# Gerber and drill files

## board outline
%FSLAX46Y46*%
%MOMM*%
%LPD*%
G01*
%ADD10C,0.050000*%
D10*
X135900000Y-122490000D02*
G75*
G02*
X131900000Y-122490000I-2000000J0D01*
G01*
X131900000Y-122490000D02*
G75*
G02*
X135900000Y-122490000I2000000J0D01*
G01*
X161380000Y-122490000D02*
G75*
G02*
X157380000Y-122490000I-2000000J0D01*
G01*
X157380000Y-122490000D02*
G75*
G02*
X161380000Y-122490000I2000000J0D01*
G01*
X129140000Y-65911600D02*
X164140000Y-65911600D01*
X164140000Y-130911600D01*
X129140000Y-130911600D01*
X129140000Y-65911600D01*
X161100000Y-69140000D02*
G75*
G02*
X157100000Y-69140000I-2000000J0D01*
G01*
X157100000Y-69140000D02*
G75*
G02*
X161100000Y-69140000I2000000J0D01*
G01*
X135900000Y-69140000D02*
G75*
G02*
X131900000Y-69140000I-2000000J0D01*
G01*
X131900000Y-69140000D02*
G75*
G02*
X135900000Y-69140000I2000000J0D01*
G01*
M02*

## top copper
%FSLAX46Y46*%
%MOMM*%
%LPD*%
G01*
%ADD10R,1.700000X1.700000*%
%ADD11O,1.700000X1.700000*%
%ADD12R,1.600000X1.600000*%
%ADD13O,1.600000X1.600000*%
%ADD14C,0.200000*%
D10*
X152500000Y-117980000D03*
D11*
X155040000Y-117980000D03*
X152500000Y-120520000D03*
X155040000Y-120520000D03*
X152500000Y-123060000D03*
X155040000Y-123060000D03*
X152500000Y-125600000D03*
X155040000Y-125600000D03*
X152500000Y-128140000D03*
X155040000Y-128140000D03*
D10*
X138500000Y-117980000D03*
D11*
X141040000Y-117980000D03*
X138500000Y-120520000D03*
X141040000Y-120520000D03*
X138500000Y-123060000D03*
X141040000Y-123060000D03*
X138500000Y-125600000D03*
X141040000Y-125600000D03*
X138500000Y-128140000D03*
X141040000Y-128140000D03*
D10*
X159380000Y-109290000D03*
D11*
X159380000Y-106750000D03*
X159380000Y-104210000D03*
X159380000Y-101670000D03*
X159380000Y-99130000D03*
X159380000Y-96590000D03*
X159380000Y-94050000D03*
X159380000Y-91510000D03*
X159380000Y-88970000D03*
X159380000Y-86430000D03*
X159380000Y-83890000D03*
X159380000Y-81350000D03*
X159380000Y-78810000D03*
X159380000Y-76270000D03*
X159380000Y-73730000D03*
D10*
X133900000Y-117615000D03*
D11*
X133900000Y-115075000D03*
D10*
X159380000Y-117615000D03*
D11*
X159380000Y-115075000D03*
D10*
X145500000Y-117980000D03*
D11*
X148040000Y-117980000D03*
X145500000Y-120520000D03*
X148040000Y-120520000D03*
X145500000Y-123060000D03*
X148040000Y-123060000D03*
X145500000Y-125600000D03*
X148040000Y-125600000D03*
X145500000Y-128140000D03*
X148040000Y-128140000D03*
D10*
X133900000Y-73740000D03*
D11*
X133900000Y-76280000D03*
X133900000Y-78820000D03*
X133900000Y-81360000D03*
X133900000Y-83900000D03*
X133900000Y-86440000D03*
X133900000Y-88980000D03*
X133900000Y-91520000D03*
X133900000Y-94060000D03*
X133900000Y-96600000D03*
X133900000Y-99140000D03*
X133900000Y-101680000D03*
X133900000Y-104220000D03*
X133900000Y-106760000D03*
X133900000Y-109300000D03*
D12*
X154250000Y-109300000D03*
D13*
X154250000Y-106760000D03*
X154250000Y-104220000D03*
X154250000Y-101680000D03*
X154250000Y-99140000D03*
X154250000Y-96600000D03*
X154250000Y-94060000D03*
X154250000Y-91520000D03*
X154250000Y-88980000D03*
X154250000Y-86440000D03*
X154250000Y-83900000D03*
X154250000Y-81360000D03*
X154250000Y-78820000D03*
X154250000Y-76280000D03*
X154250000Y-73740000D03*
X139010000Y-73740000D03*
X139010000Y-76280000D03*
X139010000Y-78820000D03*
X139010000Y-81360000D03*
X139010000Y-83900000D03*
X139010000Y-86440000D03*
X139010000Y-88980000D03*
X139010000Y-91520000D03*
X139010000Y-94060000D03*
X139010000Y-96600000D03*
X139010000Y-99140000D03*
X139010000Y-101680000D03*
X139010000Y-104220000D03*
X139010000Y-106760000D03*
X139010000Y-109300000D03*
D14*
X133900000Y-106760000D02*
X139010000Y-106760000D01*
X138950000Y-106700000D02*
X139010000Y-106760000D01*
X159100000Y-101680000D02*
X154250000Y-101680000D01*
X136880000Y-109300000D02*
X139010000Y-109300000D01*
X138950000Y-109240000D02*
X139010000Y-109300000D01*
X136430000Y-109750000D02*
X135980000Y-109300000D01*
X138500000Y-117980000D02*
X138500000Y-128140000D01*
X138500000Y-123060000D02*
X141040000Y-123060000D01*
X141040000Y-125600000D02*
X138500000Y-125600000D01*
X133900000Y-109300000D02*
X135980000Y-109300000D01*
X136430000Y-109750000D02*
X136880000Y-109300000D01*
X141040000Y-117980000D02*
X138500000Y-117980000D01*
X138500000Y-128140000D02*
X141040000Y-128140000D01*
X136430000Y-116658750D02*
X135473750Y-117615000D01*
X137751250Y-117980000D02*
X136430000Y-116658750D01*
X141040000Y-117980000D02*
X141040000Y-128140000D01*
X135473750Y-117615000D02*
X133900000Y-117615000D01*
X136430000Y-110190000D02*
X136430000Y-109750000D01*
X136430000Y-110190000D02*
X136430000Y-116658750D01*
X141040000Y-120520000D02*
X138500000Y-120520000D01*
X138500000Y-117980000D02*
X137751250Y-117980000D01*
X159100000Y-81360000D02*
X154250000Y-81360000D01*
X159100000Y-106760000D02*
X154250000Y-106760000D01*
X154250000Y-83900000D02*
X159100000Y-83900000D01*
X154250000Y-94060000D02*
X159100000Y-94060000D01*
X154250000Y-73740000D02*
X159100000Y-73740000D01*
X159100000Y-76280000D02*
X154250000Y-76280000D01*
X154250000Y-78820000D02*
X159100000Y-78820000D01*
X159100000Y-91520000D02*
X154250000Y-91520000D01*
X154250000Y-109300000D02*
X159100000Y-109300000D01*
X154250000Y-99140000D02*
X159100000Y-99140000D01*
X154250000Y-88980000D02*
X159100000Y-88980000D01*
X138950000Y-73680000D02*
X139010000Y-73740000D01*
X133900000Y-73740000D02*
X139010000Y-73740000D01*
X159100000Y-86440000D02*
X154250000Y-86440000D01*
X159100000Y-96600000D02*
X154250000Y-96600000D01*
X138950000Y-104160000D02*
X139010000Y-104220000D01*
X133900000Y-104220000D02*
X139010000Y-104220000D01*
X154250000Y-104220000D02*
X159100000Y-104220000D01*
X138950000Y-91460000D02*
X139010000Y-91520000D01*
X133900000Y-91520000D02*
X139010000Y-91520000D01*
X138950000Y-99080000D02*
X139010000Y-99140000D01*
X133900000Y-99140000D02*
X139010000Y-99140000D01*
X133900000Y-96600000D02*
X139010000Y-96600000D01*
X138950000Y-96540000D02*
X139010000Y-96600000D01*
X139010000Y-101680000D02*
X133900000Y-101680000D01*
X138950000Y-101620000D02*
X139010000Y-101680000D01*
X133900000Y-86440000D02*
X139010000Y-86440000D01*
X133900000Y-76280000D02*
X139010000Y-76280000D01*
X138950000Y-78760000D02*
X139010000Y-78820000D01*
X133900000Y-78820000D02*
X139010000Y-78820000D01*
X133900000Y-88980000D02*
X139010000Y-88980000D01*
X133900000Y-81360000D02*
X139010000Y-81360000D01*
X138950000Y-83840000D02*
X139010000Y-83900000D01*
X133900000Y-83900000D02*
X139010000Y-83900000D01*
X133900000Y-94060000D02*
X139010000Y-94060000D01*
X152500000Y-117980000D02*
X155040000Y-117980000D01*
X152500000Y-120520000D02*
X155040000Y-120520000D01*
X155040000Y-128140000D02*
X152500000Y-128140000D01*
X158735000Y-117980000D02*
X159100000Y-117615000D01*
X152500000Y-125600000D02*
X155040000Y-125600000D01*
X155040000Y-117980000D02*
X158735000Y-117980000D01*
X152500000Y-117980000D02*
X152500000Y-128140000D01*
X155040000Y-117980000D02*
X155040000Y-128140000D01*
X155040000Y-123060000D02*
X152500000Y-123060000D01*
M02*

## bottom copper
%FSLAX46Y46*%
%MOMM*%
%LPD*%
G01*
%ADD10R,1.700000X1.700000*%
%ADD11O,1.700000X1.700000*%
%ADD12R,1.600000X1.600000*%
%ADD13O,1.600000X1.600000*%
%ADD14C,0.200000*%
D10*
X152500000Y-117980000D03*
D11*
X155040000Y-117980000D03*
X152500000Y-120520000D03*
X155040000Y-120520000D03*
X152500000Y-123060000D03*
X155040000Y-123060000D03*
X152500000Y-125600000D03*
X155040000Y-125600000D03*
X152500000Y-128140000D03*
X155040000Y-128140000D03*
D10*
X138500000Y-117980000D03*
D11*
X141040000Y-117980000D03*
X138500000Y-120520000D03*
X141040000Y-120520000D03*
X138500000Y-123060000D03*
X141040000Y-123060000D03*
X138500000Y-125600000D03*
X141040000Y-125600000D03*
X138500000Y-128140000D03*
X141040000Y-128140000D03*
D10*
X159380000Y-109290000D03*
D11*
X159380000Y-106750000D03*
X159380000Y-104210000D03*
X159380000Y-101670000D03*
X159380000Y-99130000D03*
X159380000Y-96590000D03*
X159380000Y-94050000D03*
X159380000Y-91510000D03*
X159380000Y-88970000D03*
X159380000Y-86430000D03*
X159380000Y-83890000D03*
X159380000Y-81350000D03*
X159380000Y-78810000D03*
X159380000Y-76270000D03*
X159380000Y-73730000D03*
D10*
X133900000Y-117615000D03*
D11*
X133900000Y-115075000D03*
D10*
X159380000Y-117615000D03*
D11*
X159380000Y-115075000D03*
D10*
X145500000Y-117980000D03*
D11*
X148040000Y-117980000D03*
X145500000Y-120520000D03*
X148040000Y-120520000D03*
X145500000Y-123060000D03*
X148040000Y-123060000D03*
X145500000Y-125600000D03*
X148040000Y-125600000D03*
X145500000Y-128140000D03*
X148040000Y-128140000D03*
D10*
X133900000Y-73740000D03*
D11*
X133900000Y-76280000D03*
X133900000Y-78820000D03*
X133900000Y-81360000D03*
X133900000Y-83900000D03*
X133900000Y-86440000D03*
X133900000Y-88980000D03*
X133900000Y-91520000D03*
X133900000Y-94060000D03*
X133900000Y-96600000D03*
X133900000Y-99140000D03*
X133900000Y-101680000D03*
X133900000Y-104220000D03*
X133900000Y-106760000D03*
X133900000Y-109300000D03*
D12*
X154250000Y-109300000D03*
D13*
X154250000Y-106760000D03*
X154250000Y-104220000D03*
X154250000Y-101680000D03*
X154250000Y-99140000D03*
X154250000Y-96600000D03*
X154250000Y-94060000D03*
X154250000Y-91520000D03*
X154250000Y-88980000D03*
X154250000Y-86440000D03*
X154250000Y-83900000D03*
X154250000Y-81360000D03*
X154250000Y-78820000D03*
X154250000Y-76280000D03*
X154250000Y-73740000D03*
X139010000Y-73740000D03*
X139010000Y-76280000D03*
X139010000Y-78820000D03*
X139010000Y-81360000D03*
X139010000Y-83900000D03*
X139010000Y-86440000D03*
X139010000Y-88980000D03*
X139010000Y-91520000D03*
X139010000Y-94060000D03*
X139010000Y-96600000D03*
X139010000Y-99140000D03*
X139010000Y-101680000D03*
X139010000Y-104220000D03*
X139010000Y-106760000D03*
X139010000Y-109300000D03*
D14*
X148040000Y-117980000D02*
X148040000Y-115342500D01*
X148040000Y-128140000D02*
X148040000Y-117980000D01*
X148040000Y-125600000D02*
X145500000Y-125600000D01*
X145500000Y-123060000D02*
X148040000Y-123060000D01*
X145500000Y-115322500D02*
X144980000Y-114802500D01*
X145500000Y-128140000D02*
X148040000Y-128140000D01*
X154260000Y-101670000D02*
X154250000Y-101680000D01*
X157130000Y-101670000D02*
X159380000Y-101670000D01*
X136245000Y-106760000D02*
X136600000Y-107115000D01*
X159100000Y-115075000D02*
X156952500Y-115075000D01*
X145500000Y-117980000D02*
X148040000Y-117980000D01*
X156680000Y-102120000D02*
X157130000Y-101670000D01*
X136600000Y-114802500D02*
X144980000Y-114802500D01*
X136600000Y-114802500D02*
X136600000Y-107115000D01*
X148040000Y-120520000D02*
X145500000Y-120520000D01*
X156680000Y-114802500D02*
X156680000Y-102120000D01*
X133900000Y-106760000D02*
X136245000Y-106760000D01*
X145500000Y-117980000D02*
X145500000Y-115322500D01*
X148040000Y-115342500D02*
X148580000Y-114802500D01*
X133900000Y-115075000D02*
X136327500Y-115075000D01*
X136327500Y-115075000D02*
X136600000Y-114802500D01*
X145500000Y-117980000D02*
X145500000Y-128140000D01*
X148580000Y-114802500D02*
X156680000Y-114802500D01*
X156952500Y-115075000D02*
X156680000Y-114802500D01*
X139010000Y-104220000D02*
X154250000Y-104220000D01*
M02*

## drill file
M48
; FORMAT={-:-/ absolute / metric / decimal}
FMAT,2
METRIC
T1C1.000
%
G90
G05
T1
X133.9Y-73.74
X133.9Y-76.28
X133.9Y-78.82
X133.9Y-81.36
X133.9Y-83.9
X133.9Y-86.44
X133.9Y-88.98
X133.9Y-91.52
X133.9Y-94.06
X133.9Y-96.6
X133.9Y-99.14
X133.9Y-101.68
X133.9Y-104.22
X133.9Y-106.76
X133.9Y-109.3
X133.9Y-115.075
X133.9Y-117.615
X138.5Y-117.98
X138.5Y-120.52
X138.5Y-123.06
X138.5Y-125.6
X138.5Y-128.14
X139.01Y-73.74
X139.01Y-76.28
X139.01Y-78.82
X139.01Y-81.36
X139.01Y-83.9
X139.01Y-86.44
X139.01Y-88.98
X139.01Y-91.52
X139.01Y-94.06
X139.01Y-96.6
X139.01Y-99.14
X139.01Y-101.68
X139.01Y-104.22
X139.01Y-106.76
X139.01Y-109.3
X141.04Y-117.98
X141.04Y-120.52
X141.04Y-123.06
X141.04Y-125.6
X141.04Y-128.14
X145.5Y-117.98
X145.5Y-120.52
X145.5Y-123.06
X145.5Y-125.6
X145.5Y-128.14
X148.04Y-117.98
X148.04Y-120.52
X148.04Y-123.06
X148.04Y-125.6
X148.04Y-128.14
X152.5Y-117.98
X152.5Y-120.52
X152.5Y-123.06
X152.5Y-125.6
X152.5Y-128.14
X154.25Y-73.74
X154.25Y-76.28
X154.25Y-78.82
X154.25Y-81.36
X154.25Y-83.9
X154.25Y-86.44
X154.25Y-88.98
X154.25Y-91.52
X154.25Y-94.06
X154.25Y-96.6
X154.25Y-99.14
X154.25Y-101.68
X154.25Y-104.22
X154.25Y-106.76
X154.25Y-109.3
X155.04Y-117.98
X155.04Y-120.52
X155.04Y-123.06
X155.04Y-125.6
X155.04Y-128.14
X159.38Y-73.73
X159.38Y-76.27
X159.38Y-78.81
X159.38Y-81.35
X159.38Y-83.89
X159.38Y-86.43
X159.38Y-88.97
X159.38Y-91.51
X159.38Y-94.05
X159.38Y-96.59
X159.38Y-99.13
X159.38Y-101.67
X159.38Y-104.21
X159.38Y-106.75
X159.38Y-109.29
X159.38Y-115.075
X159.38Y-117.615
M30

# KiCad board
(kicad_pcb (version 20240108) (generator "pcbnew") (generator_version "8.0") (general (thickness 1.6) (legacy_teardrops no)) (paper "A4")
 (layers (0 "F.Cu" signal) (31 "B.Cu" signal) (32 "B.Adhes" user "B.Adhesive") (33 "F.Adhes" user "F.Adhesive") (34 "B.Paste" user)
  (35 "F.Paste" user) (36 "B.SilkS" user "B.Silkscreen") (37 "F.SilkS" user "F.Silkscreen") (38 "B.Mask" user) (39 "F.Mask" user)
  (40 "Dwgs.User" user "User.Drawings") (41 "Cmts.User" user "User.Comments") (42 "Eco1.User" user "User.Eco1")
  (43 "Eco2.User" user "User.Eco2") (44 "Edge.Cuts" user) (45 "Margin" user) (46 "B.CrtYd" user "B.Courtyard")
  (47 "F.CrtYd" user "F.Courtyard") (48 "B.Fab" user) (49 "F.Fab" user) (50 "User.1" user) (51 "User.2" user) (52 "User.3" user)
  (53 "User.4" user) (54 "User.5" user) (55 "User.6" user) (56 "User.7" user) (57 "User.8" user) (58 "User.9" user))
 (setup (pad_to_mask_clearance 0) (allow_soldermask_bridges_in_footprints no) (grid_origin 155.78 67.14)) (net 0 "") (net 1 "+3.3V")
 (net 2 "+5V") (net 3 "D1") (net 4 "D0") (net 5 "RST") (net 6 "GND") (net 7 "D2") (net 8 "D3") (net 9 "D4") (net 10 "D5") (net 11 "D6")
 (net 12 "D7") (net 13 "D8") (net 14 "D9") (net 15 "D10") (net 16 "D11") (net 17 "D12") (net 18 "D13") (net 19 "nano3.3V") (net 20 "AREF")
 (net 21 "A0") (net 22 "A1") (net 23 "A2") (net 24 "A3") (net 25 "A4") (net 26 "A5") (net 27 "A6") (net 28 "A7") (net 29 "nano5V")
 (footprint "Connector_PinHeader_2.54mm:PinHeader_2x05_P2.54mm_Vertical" (layer "F.Cu") (at 152.5 117.98)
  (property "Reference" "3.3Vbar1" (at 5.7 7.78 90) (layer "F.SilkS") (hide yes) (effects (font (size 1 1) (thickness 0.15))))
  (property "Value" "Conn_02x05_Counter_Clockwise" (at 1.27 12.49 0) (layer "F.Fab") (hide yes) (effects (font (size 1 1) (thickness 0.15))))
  (pad "1" thru_hole rect (at 0 0) (size 1.7 1.7) (drill 1) (layers "*.Cu" "*.Mask") (remove_unused_layers no) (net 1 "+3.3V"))
  (pad "2" thru_hole oval (at 2.54 0) (size 1.7 1.7) (drill 1) (layers "*.Cu" "*.Mask") (remove_unused_layers no) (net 1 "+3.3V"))
  (pad "3" thru_hole oval (at 0 2.54) (size 1.7 1.7) (drill 1) (layers "*.Cu" "*.Mask") (remove_unused_layers no) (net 1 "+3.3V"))
  (pad "4" thru_hole oval (at 2.54 2.54) (size 1.7 1.7) (drill 1) (layers "*.Cu" "*.Mask") (remove_unused_layers no) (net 1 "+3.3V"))
  (pad "5" thru_hole oval (at 0 5.08) (size 1.7 1.7) (drill 1) (layers "*.Cu" "*.Mask") (remove_unused_layers no) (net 1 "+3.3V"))
  (pad "6" thru_hole oval (at 2.54 5.08) (size 1.7 1.7) (drill 1) (layers "*.Cu" "*.Mask") (remove_unused_layers no) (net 1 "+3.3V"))
  (pad "7" thru_hole oval (at 0 7.62) (size 1.7 1.7) (drill 1) (layers "*.Cu" "*.Mask") (remove_unused_layers no) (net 1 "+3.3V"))
  (pad "8" thru_hole oval (at 2.54 7.62) (size 1.7 1.7) (drill 1) (layers "*.Cu" "*.Mask") (remove_unused_layers no) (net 1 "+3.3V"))
  (pad "9" thru_hole oval (at 0 10.16) (size 1.7 1.7) (drill 1) (layers "*.Cu" "*.Mask") (remove_unused_layers no) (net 1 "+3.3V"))
  (pad "10" thru_hole oval (at 2.54 10.16) (size 1.7 1.7) (drill 1) (layers "*.Cu" "*.Mask") (remove_unused_layers no) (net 1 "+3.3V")))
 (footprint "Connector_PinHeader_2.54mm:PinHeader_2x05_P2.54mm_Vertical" (layer "F.Cu") (at 138.5 117.98)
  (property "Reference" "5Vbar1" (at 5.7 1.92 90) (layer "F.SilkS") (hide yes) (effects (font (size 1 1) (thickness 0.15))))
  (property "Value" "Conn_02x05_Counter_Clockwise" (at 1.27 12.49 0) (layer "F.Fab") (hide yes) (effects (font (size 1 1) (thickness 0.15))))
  (pad "1" thru_hole rect (at 0 0) (size 1.7 1.7) (drill 1) (layers "*.Cu" "*.Mask") (remove_unused_layers no) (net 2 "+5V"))
  (pad "2" thru_hole oval (at 2.54 0) (size 1.7 1.7) (drill 1) (layers "*.Cu" "*.Mask") (remove_unused_layers no) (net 2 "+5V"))
  (pad "3" thru_hole oval (at 0 2.54) (size 1.7 1.7) (drill 1) (layers "*.Cu" "*.Mask") (remove_unused_layers no) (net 2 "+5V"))
  (pad "4" thru_hole oval (at 2.54 2.54) (size 1.7 1.7) (drill 1) (layers "*.Cu" "*.Mask") (remove_unused_layers no) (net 2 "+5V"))
  (pad "5" thru_hole oval (at 0 5.08) (size 1.7 1.7) (drill 1) (layers "*.Cu" "*.Mask") (remove_unused_layers no) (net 2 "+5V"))
  (pad "6" thru_hole oval (at 2.54 5.08) (size 1.7 1.7) (drill 1) (layers "*.Cu" "*.Mask") (remove_unused_layers no) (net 2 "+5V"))
  (pad "7" thru_hole oval (at 0 7.62) (size 1.7 1.7) (drill 1) (layers "*.Cu" "*.Mask") (remove_unused_layers no) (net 2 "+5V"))
  (pad "8" thru_hole oval (at 2.54 7.62) (size 1.7 1.7) (drill 1) (layers "*.Cu" "*.Mask") (remove_unused_layers no) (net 2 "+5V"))
  (pad "9" thru_hole oval (at 0 10.16) (size 1.7 1.7) (drill 1) (layers "*.Cu" "*.Mask") (remove_unused_layers no) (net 2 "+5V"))
  (pad "10" thru_hole oval (at 2.54 10.16) (size 1.7 1.7) (drill 1) (layers "*.Cu" "*.Mask") (remove_unused_layers no) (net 2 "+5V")))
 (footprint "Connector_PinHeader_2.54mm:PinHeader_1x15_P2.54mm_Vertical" (layer "F.Cu") (at 159.38 109.29 180)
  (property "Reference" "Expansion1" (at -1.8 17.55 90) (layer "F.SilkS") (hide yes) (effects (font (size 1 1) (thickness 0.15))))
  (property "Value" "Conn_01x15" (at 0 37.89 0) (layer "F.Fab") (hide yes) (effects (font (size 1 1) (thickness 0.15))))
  (pad "1" thru_hole rect (at 0 0 180) (size 1.7 1.7) (drill 1) (layers "*.Cu" "*.Mask") (remove_unused_layers no) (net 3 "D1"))
  (pad "2" thru_hole oval (at 0 2.54 180) (size 1.7 1.7) (drill 1) (layers "*.Cu" "*.Mask") (remove_unused_layers no) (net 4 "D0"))
  (pad "3" thru_hole oval (at 0 5.08 180) (size 1.7 1.7) (drill 1) (layers "*.Cu" "*.Mask") (remove_unused_layers no) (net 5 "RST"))
  (pad "4" thru_hole oval (at 0 7.62 180) (size 1.7 1.7) (drill 1) (layers "*.Cu" "*.Mask") (remove_unused_layers no) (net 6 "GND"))
  (pad "5" thru_hole oval (at 0 10.16 180) (size 1.7 1.7) (drill 1) (layers "*.Cu" "*.Mask") (remove_unused_layers no) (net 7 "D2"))
  (pad "6" thru_hole oval (at 0 12.7 180) (size 1.7 1.7) (drill 1) (layers "*.Cu" "*.Mask") (remove_unused_layers no) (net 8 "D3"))
  (pad "7" thru_hole oval (at 0 15.24 180) (size 1.7 1.7) (drill 1) (layers "*.Cu" "*.Mask") (remove_unused_layers no) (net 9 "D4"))
  (pad "8" thru_hole oval (at 0 17.78 180) (size 1.7 1.7) (drill 1) (layers "*.Cu" "*.Mask") (remove_unused_layers no) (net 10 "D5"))
  (pad "9" thru_hole oval (at 0 20.32 180) (size 1.7 1.7) (drill 1) (layers "*.Cu" "*.Mask") (remove_unused_layers no) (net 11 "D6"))
  (pad "10" thru_hole oval (at 0 22.86 180) (size 1.7 1.7) (drill 1) (layers "*.Cu" "*.Mask") (remove_unused_layers no) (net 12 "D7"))
  (pad "11" thru_hole oval (at 0 25.4 180) (size 1.7 1.7) (drill 1) (layers "*.Cu" "*.Mask") (remove_unused_layers no) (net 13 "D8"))
  (pad "12" thru_hole oval (at 0 27.94 180) (size 1.7 1.7) (drill 1) (layers "*.Cu" "*.Mask") (remove_unused_layers no) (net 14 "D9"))
  (pad "13" thru_hole oval (at 0 30.48 180) (size 1.7 1.7) (drill 1) (layers "*.Cu" "*.Mask") (remove_unused_layers no) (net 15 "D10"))
  (pad "14" thru_hole oval (at 0 33.02 180) (size 1.7 1.7) (drill 1) (layers "*.Cu" "*.Mask") (remove_unused_layers no) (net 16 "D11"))
  (pad "15" thru_hole oval (at 0 35.56 180) (size 1.7 1.7) (drill 1) (layers "*.Cu" "*.Mask") (remove_unused_layers no) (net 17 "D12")))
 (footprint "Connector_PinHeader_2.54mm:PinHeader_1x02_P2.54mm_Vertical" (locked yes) (layer "F.Cu") (at 133.9 117.615 180)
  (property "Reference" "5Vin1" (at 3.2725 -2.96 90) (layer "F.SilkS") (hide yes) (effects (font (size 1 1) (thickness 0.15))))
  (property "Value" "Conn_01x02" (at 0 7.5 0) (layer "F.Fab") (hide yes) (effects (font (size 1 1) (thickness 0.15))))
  (pad "1" thru_hole rect (at 0 0 180) (size 1.7 1.7) (drill 1) (layers "*.Cu" "*.Mask") (remove_unused_layers no) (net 2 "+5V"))
  (pad "2" thru_hole oval (at 0 2.54 180) (size 1.7 1.7) (drill 1) (layers "*.Cu" "*.Mask") (remove_unused_layers no) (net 6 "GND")))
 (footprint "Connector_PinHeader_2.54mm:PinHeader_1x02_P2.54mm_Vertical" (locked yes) (layer "F.Cu") (at 159.38 117.615 180)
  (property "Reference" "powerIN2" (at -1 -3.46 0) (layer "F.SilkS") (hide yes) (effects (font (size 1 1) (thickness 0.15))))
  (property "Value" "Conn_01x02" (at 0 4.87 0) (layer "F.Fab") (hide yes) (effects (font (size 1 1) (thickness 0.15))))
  (pad "1" thru_hole rect (at 0 0 180) (size 1.7 1.7) (drill 1) (layers "*.Cu" "*.Mask") (remove_unused_layers no) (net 1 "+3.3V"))
  (pad "2" thru_hole oval (at 0 2.54 180) (size 1.7 1.7) (drill 1) (layers "*.Cu" "*.Mask") (remove_unused_layers no) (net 6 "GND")))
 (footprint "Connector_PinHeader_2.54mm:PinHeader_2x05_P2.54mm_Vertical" (layer "F.Cu") (at 145.5 117.98)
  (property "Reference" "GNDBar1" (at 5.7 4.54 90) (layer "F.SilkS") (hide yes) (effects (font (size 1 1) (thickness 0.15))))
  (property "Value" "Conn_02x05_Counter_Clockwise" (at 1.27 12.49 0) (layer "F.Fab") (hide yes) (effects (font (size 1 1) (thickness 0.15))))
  (pad "1" thru_hole rect (at 0 0) (size 1.7 1.7) (drill 1) (layers "*.Cu" "*.Mask") (remove_unused_layers no) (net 6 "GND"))
  (pad "2" thru_hole oval (at 2.54 0) (size 1.7 1.7) (drill 1) (layers "*.Cu" "*.Mask") (remove_unused_layers no) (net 6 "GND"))
  (pad "3" thru_hole oval (at 0 2.54) (size 1.7 1.7) (drill 1) (layers "*.Cu" "*.Mask") (remove_unused_layers no) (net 6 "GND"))
  (pad "4" thru_hole oval (at 2.54 2.54) (size 1.7 1.7) (drill 1) (layers "*.Cu" "*.Mask") (remove_unused_layers no) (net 6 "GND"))
  (pad "5" thru_hole oval (at 0 5.08) (size 1.7 1.7) (drill 1) (layers "*.Cu" "*.Mask") (remove_unused_layers no) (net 6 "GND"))
  (pad "6" thru_hole oval (at 2.54 5.08) (size 1.7 1.7) (drill 1) (layers "*.Cu" "*.Mask") (remove_unused_layers no) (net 6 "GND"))
  (pad "7" thru_hole oval (at 0 7.62) (size 1.7 1.7) (drill 1) (layers "*.Cu" "*.Mask") (remove_unused_layers no) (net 6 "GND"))
  (pad "8" thru_hole oval (at 2.54 7.62) (size 1.7 1.7) (drill 1) (layers "*.Cu" "*.Mask") (remove_unused_layers no) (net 6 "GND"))
  (pad "9" thru_hole oval (at 0 10.16) (size 1.7 1.7) (drill 1) (layers "*.Cu" "*.Mask") (remove_unused_layers no) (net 6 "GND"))
  (pad "10" thru_hole oval (at 2.54 10.16) (size 1.7 1.7) (drill 1) (layers "*.Cu" "*.Mask") (remove_unused_layers no) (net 6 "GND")))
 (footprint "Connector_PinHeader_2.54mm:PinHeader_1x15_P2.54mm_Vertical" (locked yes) (layer "F.Cu") (at 133.9 73.74)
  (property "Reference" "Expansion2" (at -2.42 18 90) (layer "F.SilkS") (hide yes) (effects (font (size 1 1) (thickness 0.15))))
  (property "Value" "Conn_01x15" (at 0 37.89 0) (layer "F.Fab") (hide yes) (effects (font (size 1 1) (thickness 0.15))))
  (pad "1" thru_hole rect (at 0 0) (size 1.7 1.7) (drill 1) (layers "*.Cu" "*.Mask") (remove_unused_layers no) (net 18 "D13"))
  (pad "2" thru_hole oval (at 0 2.54) (size 1.7 1.7) (drill 1) (layers "*.Cu" "*.Mask") (remove_unused_layers no) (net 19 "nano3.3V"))
  (pad "3" thru_hole oval (at 0 5.08) (size 1.7 1.7) (drill 1) (layers "*.Cu" "*.Mask") (remove_unused_layers no) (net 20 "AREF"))
  (pad "4" thru_hole oval (at 0 7.62) (size 1.7 1.7) (drill 1) (layers "*.Cu" "*.Mask") (remove_unused_layers no) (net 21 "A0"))
  (pad "5" thru_hole oval (at 0 10.16) (size 1.7 1.7) (drill 1) (layers "*.Cu" "*.Mask") (remove_unused_layers no) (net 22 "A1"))
  (pad "6" thru_hole oval (at 0 12.7) (size 1.7 1.7) (drill 1) (layers "*.Cu" "*.Mask") (remove_unused_layers no) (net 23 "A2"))
  (pad "7" thru_hole oval (at 0 15.24) (size 1.7 1.7) (drill 1) (layers "*.Cu" "*.Mask") (remove_unused_layers no) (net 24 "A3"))
  (pad "8" thru_hole oval (at 0 17.78) (size 1.7 1.7) (drill 1) (layers "*.Cu" "*.Mask") (remove_unused_layers no) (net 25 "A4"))
  (pad "9" thru_hole oval (at 0 20.32) (size 1.7 1.7) (drill 1) (layers "*.Cu" "*.Mask") (remove_unused_layers no) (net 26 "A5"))
  (pad "10" thru_hole oval (at 0 22.86) (size 1.7 1.7) (drill 1) (layers "*.Cu" "*.Mask") (remove_unused_layers no) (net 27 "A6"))
  (pad "11" thru_hole oval (at 0 25.4) (size 1.7 1.7) (drill 1) (layers "*.Cu" "*.Mask") (remove_unused_layers no) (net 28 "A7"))
  (pad "12" thru_hole oval (at 0 27.94) (size 1.7 1.7) (drill 1) (layers "*.Cu" "*.Mask") (remove_unused_layers no) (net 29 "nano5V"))
  (pad "13" thru_hole oval (at 0 30.48) (size 1.7 1.7) (drill 1) (layers "*.Cu" "*.Mask") (remove_unused_layers no) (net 5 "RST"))
  (pad "14" thru_hole oval (at 0 33.02) (size 1.7 1.7) (drill 1) (layers "*.Cu" "*.Mask") (remove_unused_layers no) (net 6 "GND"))
  (pad "15" thru_hole oval (at 0 35.56) (size 1.7 1.7) (drill 1) (layers "*.Cu" "*.Mask") (remove_unused_layers no) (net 2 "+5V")))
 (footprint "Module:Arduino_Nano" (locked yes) (layer "F.Cu") (at 154.25 109.3 180)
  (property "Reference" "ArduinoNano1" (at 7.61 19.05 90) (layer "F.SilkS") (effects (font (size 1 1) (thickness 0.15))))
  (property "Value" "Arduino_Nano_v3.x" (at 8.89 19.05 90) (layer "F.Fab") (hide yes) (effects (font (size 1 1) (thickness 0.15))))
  (pad "1" thru_hole rect (at 0 0 180) (size 1.6 1.6) (drill 1) (layers "*.Cu" "*.Mask") (remove_unused_layers no) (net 3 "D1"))
  (pad "2" thru_hole oval (at 0 2.54 180) (size 1.6 1.6) (drill 1) (layers "*.Cu" "*.Mask") (remove_unused_layers no) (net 4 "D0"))
  (pad "3" thru_hole oval (at 0 5.08 180) (size 1.6 1.6) (drill 1) (layers "*.Cu" "*.Mask") (remove_unused_layers no) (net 5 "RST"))
  (pad "4" thru_hole oval (at 0 7.62 180) (size 1.6 1.6) (drill 1) (layers "*.Cu" "*.Mask") (remove_unused_layers no) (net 6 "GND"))
  (pad "5" thru_hole oval (at 0 10.16 180) (size 1.6 1.6) (drill 1) (layers "*.Cu" "*.Mask") (remove_unused_layers no) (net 7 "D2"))
  (pad "6" thru_hole oval (at 0 12.7 180) (size 1.6 1.6) (drill 1) (layers "*.Cu" "*.Mask") (remove_unused_layers no) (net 8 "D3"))
  (pad "7" thru_hole oval (at 0 15.24 180) (size 1.6 1.6) (drill 1) (layers "*.Cu" "*.Mask") (remove_unused_layers no) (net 9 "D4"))
  (pad "8" thru_hole oval (at 0 17.78 180) (size 1.6 1.6) (drill 1) (layers "*.Cu" "*.Mask") (remove_unused_layers no) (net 10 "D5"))
  (pad "9" thru_hole oval (at 0 20.32 180) (size 1.6 1.6) (drill 1) (layers "*.Cu" "*.Mask") (remove_unused_layers no) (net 11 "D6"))
  (pad "10" thru_hole oval (at 0 22.86 180) (size 1.6 1.6) (drill 1) (layers "*.Cu" "*.Mask") (remove_unused_layers no) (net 12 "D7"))
  (pad "11" thru_hole oval (at 0 25.4 180) (size 1.6 1.6) (drill 1) (layers "*.Cu" "*.Mask") (remove_unused_layers no) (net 13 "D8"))
  (pad "12" thru_hole oval (at 0 27.94 180) (size 1.6 1.6) (drill 1) (layers "*.Cu" "*.Mask") (remove_unused_layers no) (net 14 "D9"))
  (pad "13" thru_hole oval (at 0 30.48 180) (size 1.6 1.6) (drill 1) (layers "*.Cu" "*.Mask") (remove_unused_layers no) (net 15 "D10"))
  (pad "14" thru_hole oval (at 0 33.02 180) (size 1.6 1.6) (drill 1) (layers "*.Cu" "*.Mask") (remove_unused_layers no) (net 16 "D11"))
  (pad "15" thru_hole oval (at 0 35.56 180) (size 1.6 1.6) (drill 1) (layers "*.Cu" "*.Mask") (remove_unused_layers no) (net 17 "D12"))
  (pad "16" thru_hole oval (at 15.24 35.56 180) (size 1.6 1.6) (drill 1) (layers "*.Cu" "*.Mask") (remove_unused_layers no) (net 18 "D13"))
  (pad "17" thru_hole oval (at 15.24 33.02 180) (size 1.6 1.6) (drill 1) (layers "*.Cu" "*.Mask") (remove_unused_layers no)
   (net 19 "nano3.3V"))
  (pad "18" thru_hole oval (at 15.24 30.48 180) (size 1.6 1.6) (drill 1) (layers "*.Cu" "*.Mask") (remove_unused_layers no) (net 20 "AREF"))
  (pad "19" thru_hole oval (at 15.24 27.94 180) (size 1.6 1.6) (drill 1) (layers "*.Cu" "*.Mask") (remove_unused_layers no) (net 21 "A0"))
  (pad "20" thru_hole oval (at 15.24 25.4 180) (size 1.6 1.6) (drill 1) (layers "*.Cu" "*.Mask") (remove_unused_layers no) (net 22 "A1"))
  (pad "21" thru_hole oval (at 15.24 22.86 180) (size 1.6 1.6) (drill 1) (layers "*.Cu" "*.Mask") (remove_unused_layers no) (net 23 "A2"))
  (pad "22" thru_hole oval (at 15.24 20.32 180) (size 1.6 1.6) (drill 1) (layers "*.Cu" "*.Mask") (remove_unused_layers no) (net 24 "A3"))
  (pad "23" thru_hole oval (at 15.24 17.78 180) (size 1.6 1.6) (drill 1) (layers "*.Cu" "*.Mask") (remove_unused_layers no) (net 25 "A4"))
  (pad "24" thru_hole oval (at 15.24 15.24 180) (size 1.6 1.6) (drill 1) (layers "*.Cu" "*.Mask") (remove_unused_layers no) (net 26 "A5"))
  (pad "25" thru_hole oval (at 15.24 12.7 180) (size 1.6 1.6) (drill 1) (layers "*.Cu" "*.Mask") (remove_unused_layers no) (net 27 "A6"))
  (pad "26" thru_hole oval (at 15.24 10.16 180) (size 1.6 1.6) (drill 1) (layers "*.Cu" "*.Mask") (remove_unused_layers no) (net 28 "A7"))
  (pad "27" thru_hole oval (at 15.24 7.62 180) (size 1.6 1.6) (drill 1) (layers "*.Cu" "*.Mask") (remove_unused_layers no) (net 29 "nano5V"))
  (pad "28" thru_hole oval (at 15.24 5.08 180) (size 1.6 1.6) (drill 1) (layers "*.Cu" "*.Mask") (remove_unused_layers no) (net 5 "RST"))
  (pad "29" thru_hole oval (at 15.24 2.54 180) (size 1.6 1.6) (drill 1) (layers "*.Cu" "*.Mask") (remove_unused_layers no) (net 6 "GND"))
  (pad "30" thru_hole oval (at 15.24 0 180) (size 1.6 1.6) (drill 1) (layers "*.Cu" "*.Mask") (remove_unused_layers no) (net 2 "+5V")))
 (gr_circle (center 133.9 122.49) (end 135.9 122.49) (stroke (width 0.05) (type default)) (fill none) (layer "Edge.Cuts"))
 (gr_circle (center 159.38 122.49) (end 161.38 122.49) (stroke (width 0.05) (type default)) (fill none) (layer "Edge.Cuts"))
 (gr_rect (start 129.14 65.9116) (end 164.14 130.9116) (stroke (width 0.05) (type default)) (fill none) (layer "Edge.Cuts"))
 (gr_circle (center 159.1 69.14) (end 161.1 69.14) (stroke (width 0.05) (type default)) (fill none) (layer "Edge.Cuts"))
 (gr_circle (center 133.9 69.14) (end 135.9 69.14) (stroke (width 0.05) (type default)) (fill none) (layer "Edge.Cuts"))
 (segment (start 133.9 106.76) (end 139.01 106.76) (width 0.2) (layer "F.Cu") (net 6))
 (segment (start 138.95 106.7) (end 139.01 106.76) (width 0.2) (layer "F.Cu") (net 6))
 (segment (start 159.1 101.68) (end 154.25 101.68) (width 0.2) (layer "F.Cu") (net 6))
 (segment (start 148.04 117.98) (end 148.04 115.3425) (width 0.2) (layer "B.Cu") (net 6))
 (segment (start 148.04 128.14) (end 148.04 117.98) (width 0.2) (layer "B.Cu") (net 6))
 (segment (start 148.04 125.6) (end 145.5 125.6) (width 0.2) (layer "B.Cu") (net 6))
 (segment (start 145.5 123.06) (end 148.04 123.06) (width 0.2) (layer "B.Cu") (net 6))
 (segment (start 145.5 115.3225) (end 144.98 114.8025) (width 0.2) (layer "B.Cu") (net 6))
 (segment (start 145.5 128.14) (end 148.04 128.14) (width 0.2) (layer "B.Cu") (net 6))
 (segment (start 154.26 101.67) (end 154.25 101.68) (width 0.2) (layer "B.Cu") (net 6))
 (segment (start 157.13 101.67) (end 159.38 101.67) (width 0.2) (layer "B.Cu") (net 6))
 (segment (start 136.245 106.76) (end 136.6 107.115) (width 0.2) (layer "B.Cu") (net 6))
 (segment (start 159.1 115.075) (end 156.9525 115.075) (width 0.2) (layer "B.Cu") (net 6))
 (segment (start 145.5 117.98) (end 148.04 117.98) (width 0.2) (layer "B.Cu") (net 6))
 (segment (start 156.68 102.12) (end 157.13 101.67) (width 0.2) (layer "B.Cu") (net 6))
 (segment (start 136.6 114.8025) (end 144.98 114.8025) (width 0.2) (layer "B.Cu") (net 6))
 (segment (start 136.6 114.8025) (end 136.6 107.115) (width 0.2) (layer "B.Cu") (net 6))
 (segment (start 148.04 120.52) (end 145.5 120.52) (width 0.2) (layer "B.Cu") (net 6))
 (segment (start 156.68 114.8025) (end 156.68 102.12) (width 0.2) (layer "B.Cu") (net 6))
 (segment (start 133.9 106.76) (end 136.245 106.76) (width 0.2) (layer "B.Cu") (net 6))
 (segment (start 145.5 117.98) (end 145.5 115.3225) (width 0.2) (layer "B.Cu") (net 6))
 (segment (start 148.04 115.3425) (end 148.58 114.8025) (width 0.2) (layer "B.Cu") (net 6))
 (segment (start 133.9 115.075) (end 136.3275 115.075) (width 0.2) (layer "B.Cu") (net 6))
 (segment (start 136.3275 115.075) (end 136.6 114.8025) (width 0.2) (layer "B.Cu") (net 6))
 (segment (start 145.5 117.98) (end 145.5 128.14) (width 0.2) (layer "B.Cu") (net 6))
 (segment (start 148.58 114.8025) (end 156.68 114.8025) (width 0.2) (layer "B.Cu") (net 6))
 (segment (start 156.9525 115.075) (end 156.68 114.8025) (width 0.2) (layer "B.Cu") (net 6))
 (segment (start 136.88 109.3) (end 139.01 109.3) (width 0.2) (layer "F.Cu") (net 2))
 (segment (start 138.95 109.24) (end 139.01 109.3) (width 0.2) (layer "F.Cu") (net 2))
 (segment (start 136.43 109.75) (end 135.98 109.3) (width 0.2) (layer "F.Cu") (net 2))
 (segment (start 138.5 117.98) (end 138.5 128.14) (width 0.2) (layer "F.Cu") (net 2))
 (segment (start 138.5 123.06) (end 141.04 123.06) (width 0.2) (layer "F.Cu") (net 2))
 (segment (start 141.04 125.6) (end 138.5 125.6) (width 0.2) (layer "F.Cu") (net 2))
 (segment (start 133.9 109.3) (end 135.98 109.3) (width 0.2) (layer "F.Cu") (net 2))
 (segment (start 136.43 109.75) (end 136.88 109.3) (width 0.2) (layer "F.Cu") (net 2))
 (segment (start 141.04 117.98) (end 138.5 117.98) (width 0.2) (layer "F.Cu") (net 2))
 (segment (start 138.5 128.14) (end 141.04 128.14) (width 0.2) (layer "F.Cu") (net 2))
 (segment (start 136.43 116.65875) (end 135.47375 117.615) (width 0.2) (layer "F.Cu") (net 2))
 (segment (start 137.75125 117.98) (end 136.43 116.65875) (width 0.2) (layer "F.Cu") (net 2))
 (segment (start 141.04 117.98) (end 141.04 128.14) (width 0.2) (layer "F.Cu") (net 2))
 (segment (start 135.47375 117.615) (end 133.9 117.615) (width 0.2) (layer "F.Cu") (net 2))
 (segment (start 136.43 110.19) (end 136.43 109.75) (width 0.2) (layer "F.Cu") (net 2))
 (segment (start 136.43 110.19) (end 136.43 116.65875) (width 0.2) (layer "F.Cu") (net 2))
 (segment (start 141.04 120.52) (end 138.5 120.52) (width 0.2) (layer "F.Cu") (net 2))
 (segment (start 138.5 117.98) (end 137.75125 117.98) (width 0.2) (layer "F.Cu") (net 2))
 (segment (start 159.1 81.36) (end 154.25 81.36) (width 0.2) (layer "F.Cu") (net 14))
 (segment (start 159.1 106.76) (end 154.25 106.76) (width 0.2) (layer "F.Cu") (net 4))
 (segment (start 154.25 83.9) (end 159.1 83.9) (width 0.2) (layer "F.Cu") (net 13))
 (segment (start 154.25 94.06) (end 159.1 94.06) (width 0.2) (layer "F.Cu") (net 9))
 (segment (start 154.25 73.74) (end 159.1 73.74) (width 0.2) (layer "F.Cu") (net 17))
 (segment (start 159.1 76.28) (end 154.25 76.28) (width 0.2) (layer "F.Cu") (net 16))
 (segment (start 154.25 78.82) (end 159.1 78.82) (width 0.2) (layer "F.Cu") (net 15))
 (segment (start 159.1 91.52) (end 154.25 91.52) (width 0.2) (layer "F.Cu") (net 10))
 (segment (start 154.25 109.3) (end 159.1 109.3) (width 0.2) (layer "F.Cu") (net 3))
 (segment (start 154.25 99.14) (end 159.1 99.14) (width 0.2) (layer "F.Cu") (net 7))
 (segment (start 154.25 88.98) (end 159.1 88.98) (width 0.2) (layer "F.Cu") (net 11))
 (segment (start 138.95 73.68) (end 139.01 73.74) (width 0.2) (layer "F.Cu") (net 18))
 (segment (start 133.9 73.74) (end 139.01 73.74) (width 0.2) (layer "F.Cu") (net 18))
 (segment (start 159.1 86.44) (end 154.25 86.44) (width 0.2) (layer "F.Cu") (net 12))
 (segment (start 159.1 96.6) (end 154.25 96.6) (width 0.2) (layer "F.Cu") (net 8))
 (segment (start 138.95 104.16) (end 139.01 104.22) (width 0.2) (layer "F.Cu") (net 5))
 (segment (start 133.9 104.22) (end 139.01 104.22) (width 0.2) (layer "F.Cu") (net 5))
 (segment (start 154.25 104.22) (end 159.1 104.22) (width 0.2) (layer "F.Cu") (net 5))
 (segment (start 139.01 104.22) (end 154.25 104.22) (width 0.2) (layer "B.Cu") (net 5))
 (segment (start 138.95 91.46) (end 139.01 91.52) (width 0.2) (layer "F.Cu") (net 25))
 (segment (start 133.9 91.52) (end 139.01 91.52) (width 0.2) (layer "F.Cu") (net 25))
 (segment (start 138.95 99.08) (end 139.01 99.14) (width 0.2) (layer "F.Cu") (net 28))
 (segment (start 133.9 99.14) (end 139.01 99.14) (width 0.2) (layer "F.Cu") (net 28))
 (segment (start 133.9 96.6) (end 139.01 96.6) (width 0.2) (layer "F.Cu") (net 27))
 (segment (start 138.95 96.54) (end 139.01 96.6) (width 0.2) (layer "F.Cu") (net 27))
 (segment (start 139.01 101.68) (end 133.9 101.68) (width 0.2) (layer "F.Cu") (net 29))
 (segment (start 138.95 101.62) (end 139.01 101.68) (width 0.2) (layer "F.Cu") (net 29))
 (segment (start 133.9 86.44) (end 139.01 86.44) (width 0.2) (layer "F.Cu") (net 23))
 (segment (start 133.9 76.28) (end 139.01 76.28) (width 0.2) (layer "F.Cu") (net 19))
 (segment (start 138.95 78.76) (end 139.01 78.82) (width 0.2) (layer "F.Cu") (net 20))
 (segment (start 133.9 78.82) (end 139.01 78.82) (width 0.2) (layer "F.Cu") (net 20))
 (segment (start 133.9 88.98) (end 139.01 88.98) (width 0.2) (layer "F.Cu") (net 24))
 (segment (start 133.9 81.36) (end 139.01 81.36) (width 0.2) (layer "F.Cu") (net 21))
 (segment (start 138.95 83.84) (end 139.01 83.9) (width 0.2) (layer "F.Cu") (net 22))
 (segment (start 133.9 83.9) (end 139.01 83.9) (width 0.2) (layer "F.Cu") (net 22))
 (segment (start 133.9 94.06) (end 139.01 94.06) (width 0.2) (layer "F.Cu") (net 26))
 (segment (start 152.5 117.98) (end 155.04 117.98) (width 0.2) (layer "F.Cu") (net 1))
 (segment (start 152.5 120.52) (end 155.04 120.52) (width 0.2) (layer "F.Cu") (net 1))
 (segment (start 155.04 128.14) (end 152.5 128.14) (width 0.2) (layer "F.Cu") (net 1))
 (segment (start 158.735 117.98) (end 159.1 117.615) (width 0.2) (layer "F.Cu") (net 1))
 (segment (start 152.5 125.6) (end 155.04 125.6) (width 0.2) (layer "F.Cu") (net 1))
 (segment (start 155.04 117.98) (end 158.735 117.98) (width 0.2) (layer "F.Cu") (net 1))
 (segment (start 152.5 117.98) (end 152.5 128.14) (width 0.2) (layer "F.Cu") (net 1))
 (segment (start 155.04 117.98) (end 155.04 128.14) (width 0.2) (layer "F.Cu") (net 1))
 (segment (start 155.04 123.06) (end 152.5 123.06) (width 0.2) (layer "F.Cu") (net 1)))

